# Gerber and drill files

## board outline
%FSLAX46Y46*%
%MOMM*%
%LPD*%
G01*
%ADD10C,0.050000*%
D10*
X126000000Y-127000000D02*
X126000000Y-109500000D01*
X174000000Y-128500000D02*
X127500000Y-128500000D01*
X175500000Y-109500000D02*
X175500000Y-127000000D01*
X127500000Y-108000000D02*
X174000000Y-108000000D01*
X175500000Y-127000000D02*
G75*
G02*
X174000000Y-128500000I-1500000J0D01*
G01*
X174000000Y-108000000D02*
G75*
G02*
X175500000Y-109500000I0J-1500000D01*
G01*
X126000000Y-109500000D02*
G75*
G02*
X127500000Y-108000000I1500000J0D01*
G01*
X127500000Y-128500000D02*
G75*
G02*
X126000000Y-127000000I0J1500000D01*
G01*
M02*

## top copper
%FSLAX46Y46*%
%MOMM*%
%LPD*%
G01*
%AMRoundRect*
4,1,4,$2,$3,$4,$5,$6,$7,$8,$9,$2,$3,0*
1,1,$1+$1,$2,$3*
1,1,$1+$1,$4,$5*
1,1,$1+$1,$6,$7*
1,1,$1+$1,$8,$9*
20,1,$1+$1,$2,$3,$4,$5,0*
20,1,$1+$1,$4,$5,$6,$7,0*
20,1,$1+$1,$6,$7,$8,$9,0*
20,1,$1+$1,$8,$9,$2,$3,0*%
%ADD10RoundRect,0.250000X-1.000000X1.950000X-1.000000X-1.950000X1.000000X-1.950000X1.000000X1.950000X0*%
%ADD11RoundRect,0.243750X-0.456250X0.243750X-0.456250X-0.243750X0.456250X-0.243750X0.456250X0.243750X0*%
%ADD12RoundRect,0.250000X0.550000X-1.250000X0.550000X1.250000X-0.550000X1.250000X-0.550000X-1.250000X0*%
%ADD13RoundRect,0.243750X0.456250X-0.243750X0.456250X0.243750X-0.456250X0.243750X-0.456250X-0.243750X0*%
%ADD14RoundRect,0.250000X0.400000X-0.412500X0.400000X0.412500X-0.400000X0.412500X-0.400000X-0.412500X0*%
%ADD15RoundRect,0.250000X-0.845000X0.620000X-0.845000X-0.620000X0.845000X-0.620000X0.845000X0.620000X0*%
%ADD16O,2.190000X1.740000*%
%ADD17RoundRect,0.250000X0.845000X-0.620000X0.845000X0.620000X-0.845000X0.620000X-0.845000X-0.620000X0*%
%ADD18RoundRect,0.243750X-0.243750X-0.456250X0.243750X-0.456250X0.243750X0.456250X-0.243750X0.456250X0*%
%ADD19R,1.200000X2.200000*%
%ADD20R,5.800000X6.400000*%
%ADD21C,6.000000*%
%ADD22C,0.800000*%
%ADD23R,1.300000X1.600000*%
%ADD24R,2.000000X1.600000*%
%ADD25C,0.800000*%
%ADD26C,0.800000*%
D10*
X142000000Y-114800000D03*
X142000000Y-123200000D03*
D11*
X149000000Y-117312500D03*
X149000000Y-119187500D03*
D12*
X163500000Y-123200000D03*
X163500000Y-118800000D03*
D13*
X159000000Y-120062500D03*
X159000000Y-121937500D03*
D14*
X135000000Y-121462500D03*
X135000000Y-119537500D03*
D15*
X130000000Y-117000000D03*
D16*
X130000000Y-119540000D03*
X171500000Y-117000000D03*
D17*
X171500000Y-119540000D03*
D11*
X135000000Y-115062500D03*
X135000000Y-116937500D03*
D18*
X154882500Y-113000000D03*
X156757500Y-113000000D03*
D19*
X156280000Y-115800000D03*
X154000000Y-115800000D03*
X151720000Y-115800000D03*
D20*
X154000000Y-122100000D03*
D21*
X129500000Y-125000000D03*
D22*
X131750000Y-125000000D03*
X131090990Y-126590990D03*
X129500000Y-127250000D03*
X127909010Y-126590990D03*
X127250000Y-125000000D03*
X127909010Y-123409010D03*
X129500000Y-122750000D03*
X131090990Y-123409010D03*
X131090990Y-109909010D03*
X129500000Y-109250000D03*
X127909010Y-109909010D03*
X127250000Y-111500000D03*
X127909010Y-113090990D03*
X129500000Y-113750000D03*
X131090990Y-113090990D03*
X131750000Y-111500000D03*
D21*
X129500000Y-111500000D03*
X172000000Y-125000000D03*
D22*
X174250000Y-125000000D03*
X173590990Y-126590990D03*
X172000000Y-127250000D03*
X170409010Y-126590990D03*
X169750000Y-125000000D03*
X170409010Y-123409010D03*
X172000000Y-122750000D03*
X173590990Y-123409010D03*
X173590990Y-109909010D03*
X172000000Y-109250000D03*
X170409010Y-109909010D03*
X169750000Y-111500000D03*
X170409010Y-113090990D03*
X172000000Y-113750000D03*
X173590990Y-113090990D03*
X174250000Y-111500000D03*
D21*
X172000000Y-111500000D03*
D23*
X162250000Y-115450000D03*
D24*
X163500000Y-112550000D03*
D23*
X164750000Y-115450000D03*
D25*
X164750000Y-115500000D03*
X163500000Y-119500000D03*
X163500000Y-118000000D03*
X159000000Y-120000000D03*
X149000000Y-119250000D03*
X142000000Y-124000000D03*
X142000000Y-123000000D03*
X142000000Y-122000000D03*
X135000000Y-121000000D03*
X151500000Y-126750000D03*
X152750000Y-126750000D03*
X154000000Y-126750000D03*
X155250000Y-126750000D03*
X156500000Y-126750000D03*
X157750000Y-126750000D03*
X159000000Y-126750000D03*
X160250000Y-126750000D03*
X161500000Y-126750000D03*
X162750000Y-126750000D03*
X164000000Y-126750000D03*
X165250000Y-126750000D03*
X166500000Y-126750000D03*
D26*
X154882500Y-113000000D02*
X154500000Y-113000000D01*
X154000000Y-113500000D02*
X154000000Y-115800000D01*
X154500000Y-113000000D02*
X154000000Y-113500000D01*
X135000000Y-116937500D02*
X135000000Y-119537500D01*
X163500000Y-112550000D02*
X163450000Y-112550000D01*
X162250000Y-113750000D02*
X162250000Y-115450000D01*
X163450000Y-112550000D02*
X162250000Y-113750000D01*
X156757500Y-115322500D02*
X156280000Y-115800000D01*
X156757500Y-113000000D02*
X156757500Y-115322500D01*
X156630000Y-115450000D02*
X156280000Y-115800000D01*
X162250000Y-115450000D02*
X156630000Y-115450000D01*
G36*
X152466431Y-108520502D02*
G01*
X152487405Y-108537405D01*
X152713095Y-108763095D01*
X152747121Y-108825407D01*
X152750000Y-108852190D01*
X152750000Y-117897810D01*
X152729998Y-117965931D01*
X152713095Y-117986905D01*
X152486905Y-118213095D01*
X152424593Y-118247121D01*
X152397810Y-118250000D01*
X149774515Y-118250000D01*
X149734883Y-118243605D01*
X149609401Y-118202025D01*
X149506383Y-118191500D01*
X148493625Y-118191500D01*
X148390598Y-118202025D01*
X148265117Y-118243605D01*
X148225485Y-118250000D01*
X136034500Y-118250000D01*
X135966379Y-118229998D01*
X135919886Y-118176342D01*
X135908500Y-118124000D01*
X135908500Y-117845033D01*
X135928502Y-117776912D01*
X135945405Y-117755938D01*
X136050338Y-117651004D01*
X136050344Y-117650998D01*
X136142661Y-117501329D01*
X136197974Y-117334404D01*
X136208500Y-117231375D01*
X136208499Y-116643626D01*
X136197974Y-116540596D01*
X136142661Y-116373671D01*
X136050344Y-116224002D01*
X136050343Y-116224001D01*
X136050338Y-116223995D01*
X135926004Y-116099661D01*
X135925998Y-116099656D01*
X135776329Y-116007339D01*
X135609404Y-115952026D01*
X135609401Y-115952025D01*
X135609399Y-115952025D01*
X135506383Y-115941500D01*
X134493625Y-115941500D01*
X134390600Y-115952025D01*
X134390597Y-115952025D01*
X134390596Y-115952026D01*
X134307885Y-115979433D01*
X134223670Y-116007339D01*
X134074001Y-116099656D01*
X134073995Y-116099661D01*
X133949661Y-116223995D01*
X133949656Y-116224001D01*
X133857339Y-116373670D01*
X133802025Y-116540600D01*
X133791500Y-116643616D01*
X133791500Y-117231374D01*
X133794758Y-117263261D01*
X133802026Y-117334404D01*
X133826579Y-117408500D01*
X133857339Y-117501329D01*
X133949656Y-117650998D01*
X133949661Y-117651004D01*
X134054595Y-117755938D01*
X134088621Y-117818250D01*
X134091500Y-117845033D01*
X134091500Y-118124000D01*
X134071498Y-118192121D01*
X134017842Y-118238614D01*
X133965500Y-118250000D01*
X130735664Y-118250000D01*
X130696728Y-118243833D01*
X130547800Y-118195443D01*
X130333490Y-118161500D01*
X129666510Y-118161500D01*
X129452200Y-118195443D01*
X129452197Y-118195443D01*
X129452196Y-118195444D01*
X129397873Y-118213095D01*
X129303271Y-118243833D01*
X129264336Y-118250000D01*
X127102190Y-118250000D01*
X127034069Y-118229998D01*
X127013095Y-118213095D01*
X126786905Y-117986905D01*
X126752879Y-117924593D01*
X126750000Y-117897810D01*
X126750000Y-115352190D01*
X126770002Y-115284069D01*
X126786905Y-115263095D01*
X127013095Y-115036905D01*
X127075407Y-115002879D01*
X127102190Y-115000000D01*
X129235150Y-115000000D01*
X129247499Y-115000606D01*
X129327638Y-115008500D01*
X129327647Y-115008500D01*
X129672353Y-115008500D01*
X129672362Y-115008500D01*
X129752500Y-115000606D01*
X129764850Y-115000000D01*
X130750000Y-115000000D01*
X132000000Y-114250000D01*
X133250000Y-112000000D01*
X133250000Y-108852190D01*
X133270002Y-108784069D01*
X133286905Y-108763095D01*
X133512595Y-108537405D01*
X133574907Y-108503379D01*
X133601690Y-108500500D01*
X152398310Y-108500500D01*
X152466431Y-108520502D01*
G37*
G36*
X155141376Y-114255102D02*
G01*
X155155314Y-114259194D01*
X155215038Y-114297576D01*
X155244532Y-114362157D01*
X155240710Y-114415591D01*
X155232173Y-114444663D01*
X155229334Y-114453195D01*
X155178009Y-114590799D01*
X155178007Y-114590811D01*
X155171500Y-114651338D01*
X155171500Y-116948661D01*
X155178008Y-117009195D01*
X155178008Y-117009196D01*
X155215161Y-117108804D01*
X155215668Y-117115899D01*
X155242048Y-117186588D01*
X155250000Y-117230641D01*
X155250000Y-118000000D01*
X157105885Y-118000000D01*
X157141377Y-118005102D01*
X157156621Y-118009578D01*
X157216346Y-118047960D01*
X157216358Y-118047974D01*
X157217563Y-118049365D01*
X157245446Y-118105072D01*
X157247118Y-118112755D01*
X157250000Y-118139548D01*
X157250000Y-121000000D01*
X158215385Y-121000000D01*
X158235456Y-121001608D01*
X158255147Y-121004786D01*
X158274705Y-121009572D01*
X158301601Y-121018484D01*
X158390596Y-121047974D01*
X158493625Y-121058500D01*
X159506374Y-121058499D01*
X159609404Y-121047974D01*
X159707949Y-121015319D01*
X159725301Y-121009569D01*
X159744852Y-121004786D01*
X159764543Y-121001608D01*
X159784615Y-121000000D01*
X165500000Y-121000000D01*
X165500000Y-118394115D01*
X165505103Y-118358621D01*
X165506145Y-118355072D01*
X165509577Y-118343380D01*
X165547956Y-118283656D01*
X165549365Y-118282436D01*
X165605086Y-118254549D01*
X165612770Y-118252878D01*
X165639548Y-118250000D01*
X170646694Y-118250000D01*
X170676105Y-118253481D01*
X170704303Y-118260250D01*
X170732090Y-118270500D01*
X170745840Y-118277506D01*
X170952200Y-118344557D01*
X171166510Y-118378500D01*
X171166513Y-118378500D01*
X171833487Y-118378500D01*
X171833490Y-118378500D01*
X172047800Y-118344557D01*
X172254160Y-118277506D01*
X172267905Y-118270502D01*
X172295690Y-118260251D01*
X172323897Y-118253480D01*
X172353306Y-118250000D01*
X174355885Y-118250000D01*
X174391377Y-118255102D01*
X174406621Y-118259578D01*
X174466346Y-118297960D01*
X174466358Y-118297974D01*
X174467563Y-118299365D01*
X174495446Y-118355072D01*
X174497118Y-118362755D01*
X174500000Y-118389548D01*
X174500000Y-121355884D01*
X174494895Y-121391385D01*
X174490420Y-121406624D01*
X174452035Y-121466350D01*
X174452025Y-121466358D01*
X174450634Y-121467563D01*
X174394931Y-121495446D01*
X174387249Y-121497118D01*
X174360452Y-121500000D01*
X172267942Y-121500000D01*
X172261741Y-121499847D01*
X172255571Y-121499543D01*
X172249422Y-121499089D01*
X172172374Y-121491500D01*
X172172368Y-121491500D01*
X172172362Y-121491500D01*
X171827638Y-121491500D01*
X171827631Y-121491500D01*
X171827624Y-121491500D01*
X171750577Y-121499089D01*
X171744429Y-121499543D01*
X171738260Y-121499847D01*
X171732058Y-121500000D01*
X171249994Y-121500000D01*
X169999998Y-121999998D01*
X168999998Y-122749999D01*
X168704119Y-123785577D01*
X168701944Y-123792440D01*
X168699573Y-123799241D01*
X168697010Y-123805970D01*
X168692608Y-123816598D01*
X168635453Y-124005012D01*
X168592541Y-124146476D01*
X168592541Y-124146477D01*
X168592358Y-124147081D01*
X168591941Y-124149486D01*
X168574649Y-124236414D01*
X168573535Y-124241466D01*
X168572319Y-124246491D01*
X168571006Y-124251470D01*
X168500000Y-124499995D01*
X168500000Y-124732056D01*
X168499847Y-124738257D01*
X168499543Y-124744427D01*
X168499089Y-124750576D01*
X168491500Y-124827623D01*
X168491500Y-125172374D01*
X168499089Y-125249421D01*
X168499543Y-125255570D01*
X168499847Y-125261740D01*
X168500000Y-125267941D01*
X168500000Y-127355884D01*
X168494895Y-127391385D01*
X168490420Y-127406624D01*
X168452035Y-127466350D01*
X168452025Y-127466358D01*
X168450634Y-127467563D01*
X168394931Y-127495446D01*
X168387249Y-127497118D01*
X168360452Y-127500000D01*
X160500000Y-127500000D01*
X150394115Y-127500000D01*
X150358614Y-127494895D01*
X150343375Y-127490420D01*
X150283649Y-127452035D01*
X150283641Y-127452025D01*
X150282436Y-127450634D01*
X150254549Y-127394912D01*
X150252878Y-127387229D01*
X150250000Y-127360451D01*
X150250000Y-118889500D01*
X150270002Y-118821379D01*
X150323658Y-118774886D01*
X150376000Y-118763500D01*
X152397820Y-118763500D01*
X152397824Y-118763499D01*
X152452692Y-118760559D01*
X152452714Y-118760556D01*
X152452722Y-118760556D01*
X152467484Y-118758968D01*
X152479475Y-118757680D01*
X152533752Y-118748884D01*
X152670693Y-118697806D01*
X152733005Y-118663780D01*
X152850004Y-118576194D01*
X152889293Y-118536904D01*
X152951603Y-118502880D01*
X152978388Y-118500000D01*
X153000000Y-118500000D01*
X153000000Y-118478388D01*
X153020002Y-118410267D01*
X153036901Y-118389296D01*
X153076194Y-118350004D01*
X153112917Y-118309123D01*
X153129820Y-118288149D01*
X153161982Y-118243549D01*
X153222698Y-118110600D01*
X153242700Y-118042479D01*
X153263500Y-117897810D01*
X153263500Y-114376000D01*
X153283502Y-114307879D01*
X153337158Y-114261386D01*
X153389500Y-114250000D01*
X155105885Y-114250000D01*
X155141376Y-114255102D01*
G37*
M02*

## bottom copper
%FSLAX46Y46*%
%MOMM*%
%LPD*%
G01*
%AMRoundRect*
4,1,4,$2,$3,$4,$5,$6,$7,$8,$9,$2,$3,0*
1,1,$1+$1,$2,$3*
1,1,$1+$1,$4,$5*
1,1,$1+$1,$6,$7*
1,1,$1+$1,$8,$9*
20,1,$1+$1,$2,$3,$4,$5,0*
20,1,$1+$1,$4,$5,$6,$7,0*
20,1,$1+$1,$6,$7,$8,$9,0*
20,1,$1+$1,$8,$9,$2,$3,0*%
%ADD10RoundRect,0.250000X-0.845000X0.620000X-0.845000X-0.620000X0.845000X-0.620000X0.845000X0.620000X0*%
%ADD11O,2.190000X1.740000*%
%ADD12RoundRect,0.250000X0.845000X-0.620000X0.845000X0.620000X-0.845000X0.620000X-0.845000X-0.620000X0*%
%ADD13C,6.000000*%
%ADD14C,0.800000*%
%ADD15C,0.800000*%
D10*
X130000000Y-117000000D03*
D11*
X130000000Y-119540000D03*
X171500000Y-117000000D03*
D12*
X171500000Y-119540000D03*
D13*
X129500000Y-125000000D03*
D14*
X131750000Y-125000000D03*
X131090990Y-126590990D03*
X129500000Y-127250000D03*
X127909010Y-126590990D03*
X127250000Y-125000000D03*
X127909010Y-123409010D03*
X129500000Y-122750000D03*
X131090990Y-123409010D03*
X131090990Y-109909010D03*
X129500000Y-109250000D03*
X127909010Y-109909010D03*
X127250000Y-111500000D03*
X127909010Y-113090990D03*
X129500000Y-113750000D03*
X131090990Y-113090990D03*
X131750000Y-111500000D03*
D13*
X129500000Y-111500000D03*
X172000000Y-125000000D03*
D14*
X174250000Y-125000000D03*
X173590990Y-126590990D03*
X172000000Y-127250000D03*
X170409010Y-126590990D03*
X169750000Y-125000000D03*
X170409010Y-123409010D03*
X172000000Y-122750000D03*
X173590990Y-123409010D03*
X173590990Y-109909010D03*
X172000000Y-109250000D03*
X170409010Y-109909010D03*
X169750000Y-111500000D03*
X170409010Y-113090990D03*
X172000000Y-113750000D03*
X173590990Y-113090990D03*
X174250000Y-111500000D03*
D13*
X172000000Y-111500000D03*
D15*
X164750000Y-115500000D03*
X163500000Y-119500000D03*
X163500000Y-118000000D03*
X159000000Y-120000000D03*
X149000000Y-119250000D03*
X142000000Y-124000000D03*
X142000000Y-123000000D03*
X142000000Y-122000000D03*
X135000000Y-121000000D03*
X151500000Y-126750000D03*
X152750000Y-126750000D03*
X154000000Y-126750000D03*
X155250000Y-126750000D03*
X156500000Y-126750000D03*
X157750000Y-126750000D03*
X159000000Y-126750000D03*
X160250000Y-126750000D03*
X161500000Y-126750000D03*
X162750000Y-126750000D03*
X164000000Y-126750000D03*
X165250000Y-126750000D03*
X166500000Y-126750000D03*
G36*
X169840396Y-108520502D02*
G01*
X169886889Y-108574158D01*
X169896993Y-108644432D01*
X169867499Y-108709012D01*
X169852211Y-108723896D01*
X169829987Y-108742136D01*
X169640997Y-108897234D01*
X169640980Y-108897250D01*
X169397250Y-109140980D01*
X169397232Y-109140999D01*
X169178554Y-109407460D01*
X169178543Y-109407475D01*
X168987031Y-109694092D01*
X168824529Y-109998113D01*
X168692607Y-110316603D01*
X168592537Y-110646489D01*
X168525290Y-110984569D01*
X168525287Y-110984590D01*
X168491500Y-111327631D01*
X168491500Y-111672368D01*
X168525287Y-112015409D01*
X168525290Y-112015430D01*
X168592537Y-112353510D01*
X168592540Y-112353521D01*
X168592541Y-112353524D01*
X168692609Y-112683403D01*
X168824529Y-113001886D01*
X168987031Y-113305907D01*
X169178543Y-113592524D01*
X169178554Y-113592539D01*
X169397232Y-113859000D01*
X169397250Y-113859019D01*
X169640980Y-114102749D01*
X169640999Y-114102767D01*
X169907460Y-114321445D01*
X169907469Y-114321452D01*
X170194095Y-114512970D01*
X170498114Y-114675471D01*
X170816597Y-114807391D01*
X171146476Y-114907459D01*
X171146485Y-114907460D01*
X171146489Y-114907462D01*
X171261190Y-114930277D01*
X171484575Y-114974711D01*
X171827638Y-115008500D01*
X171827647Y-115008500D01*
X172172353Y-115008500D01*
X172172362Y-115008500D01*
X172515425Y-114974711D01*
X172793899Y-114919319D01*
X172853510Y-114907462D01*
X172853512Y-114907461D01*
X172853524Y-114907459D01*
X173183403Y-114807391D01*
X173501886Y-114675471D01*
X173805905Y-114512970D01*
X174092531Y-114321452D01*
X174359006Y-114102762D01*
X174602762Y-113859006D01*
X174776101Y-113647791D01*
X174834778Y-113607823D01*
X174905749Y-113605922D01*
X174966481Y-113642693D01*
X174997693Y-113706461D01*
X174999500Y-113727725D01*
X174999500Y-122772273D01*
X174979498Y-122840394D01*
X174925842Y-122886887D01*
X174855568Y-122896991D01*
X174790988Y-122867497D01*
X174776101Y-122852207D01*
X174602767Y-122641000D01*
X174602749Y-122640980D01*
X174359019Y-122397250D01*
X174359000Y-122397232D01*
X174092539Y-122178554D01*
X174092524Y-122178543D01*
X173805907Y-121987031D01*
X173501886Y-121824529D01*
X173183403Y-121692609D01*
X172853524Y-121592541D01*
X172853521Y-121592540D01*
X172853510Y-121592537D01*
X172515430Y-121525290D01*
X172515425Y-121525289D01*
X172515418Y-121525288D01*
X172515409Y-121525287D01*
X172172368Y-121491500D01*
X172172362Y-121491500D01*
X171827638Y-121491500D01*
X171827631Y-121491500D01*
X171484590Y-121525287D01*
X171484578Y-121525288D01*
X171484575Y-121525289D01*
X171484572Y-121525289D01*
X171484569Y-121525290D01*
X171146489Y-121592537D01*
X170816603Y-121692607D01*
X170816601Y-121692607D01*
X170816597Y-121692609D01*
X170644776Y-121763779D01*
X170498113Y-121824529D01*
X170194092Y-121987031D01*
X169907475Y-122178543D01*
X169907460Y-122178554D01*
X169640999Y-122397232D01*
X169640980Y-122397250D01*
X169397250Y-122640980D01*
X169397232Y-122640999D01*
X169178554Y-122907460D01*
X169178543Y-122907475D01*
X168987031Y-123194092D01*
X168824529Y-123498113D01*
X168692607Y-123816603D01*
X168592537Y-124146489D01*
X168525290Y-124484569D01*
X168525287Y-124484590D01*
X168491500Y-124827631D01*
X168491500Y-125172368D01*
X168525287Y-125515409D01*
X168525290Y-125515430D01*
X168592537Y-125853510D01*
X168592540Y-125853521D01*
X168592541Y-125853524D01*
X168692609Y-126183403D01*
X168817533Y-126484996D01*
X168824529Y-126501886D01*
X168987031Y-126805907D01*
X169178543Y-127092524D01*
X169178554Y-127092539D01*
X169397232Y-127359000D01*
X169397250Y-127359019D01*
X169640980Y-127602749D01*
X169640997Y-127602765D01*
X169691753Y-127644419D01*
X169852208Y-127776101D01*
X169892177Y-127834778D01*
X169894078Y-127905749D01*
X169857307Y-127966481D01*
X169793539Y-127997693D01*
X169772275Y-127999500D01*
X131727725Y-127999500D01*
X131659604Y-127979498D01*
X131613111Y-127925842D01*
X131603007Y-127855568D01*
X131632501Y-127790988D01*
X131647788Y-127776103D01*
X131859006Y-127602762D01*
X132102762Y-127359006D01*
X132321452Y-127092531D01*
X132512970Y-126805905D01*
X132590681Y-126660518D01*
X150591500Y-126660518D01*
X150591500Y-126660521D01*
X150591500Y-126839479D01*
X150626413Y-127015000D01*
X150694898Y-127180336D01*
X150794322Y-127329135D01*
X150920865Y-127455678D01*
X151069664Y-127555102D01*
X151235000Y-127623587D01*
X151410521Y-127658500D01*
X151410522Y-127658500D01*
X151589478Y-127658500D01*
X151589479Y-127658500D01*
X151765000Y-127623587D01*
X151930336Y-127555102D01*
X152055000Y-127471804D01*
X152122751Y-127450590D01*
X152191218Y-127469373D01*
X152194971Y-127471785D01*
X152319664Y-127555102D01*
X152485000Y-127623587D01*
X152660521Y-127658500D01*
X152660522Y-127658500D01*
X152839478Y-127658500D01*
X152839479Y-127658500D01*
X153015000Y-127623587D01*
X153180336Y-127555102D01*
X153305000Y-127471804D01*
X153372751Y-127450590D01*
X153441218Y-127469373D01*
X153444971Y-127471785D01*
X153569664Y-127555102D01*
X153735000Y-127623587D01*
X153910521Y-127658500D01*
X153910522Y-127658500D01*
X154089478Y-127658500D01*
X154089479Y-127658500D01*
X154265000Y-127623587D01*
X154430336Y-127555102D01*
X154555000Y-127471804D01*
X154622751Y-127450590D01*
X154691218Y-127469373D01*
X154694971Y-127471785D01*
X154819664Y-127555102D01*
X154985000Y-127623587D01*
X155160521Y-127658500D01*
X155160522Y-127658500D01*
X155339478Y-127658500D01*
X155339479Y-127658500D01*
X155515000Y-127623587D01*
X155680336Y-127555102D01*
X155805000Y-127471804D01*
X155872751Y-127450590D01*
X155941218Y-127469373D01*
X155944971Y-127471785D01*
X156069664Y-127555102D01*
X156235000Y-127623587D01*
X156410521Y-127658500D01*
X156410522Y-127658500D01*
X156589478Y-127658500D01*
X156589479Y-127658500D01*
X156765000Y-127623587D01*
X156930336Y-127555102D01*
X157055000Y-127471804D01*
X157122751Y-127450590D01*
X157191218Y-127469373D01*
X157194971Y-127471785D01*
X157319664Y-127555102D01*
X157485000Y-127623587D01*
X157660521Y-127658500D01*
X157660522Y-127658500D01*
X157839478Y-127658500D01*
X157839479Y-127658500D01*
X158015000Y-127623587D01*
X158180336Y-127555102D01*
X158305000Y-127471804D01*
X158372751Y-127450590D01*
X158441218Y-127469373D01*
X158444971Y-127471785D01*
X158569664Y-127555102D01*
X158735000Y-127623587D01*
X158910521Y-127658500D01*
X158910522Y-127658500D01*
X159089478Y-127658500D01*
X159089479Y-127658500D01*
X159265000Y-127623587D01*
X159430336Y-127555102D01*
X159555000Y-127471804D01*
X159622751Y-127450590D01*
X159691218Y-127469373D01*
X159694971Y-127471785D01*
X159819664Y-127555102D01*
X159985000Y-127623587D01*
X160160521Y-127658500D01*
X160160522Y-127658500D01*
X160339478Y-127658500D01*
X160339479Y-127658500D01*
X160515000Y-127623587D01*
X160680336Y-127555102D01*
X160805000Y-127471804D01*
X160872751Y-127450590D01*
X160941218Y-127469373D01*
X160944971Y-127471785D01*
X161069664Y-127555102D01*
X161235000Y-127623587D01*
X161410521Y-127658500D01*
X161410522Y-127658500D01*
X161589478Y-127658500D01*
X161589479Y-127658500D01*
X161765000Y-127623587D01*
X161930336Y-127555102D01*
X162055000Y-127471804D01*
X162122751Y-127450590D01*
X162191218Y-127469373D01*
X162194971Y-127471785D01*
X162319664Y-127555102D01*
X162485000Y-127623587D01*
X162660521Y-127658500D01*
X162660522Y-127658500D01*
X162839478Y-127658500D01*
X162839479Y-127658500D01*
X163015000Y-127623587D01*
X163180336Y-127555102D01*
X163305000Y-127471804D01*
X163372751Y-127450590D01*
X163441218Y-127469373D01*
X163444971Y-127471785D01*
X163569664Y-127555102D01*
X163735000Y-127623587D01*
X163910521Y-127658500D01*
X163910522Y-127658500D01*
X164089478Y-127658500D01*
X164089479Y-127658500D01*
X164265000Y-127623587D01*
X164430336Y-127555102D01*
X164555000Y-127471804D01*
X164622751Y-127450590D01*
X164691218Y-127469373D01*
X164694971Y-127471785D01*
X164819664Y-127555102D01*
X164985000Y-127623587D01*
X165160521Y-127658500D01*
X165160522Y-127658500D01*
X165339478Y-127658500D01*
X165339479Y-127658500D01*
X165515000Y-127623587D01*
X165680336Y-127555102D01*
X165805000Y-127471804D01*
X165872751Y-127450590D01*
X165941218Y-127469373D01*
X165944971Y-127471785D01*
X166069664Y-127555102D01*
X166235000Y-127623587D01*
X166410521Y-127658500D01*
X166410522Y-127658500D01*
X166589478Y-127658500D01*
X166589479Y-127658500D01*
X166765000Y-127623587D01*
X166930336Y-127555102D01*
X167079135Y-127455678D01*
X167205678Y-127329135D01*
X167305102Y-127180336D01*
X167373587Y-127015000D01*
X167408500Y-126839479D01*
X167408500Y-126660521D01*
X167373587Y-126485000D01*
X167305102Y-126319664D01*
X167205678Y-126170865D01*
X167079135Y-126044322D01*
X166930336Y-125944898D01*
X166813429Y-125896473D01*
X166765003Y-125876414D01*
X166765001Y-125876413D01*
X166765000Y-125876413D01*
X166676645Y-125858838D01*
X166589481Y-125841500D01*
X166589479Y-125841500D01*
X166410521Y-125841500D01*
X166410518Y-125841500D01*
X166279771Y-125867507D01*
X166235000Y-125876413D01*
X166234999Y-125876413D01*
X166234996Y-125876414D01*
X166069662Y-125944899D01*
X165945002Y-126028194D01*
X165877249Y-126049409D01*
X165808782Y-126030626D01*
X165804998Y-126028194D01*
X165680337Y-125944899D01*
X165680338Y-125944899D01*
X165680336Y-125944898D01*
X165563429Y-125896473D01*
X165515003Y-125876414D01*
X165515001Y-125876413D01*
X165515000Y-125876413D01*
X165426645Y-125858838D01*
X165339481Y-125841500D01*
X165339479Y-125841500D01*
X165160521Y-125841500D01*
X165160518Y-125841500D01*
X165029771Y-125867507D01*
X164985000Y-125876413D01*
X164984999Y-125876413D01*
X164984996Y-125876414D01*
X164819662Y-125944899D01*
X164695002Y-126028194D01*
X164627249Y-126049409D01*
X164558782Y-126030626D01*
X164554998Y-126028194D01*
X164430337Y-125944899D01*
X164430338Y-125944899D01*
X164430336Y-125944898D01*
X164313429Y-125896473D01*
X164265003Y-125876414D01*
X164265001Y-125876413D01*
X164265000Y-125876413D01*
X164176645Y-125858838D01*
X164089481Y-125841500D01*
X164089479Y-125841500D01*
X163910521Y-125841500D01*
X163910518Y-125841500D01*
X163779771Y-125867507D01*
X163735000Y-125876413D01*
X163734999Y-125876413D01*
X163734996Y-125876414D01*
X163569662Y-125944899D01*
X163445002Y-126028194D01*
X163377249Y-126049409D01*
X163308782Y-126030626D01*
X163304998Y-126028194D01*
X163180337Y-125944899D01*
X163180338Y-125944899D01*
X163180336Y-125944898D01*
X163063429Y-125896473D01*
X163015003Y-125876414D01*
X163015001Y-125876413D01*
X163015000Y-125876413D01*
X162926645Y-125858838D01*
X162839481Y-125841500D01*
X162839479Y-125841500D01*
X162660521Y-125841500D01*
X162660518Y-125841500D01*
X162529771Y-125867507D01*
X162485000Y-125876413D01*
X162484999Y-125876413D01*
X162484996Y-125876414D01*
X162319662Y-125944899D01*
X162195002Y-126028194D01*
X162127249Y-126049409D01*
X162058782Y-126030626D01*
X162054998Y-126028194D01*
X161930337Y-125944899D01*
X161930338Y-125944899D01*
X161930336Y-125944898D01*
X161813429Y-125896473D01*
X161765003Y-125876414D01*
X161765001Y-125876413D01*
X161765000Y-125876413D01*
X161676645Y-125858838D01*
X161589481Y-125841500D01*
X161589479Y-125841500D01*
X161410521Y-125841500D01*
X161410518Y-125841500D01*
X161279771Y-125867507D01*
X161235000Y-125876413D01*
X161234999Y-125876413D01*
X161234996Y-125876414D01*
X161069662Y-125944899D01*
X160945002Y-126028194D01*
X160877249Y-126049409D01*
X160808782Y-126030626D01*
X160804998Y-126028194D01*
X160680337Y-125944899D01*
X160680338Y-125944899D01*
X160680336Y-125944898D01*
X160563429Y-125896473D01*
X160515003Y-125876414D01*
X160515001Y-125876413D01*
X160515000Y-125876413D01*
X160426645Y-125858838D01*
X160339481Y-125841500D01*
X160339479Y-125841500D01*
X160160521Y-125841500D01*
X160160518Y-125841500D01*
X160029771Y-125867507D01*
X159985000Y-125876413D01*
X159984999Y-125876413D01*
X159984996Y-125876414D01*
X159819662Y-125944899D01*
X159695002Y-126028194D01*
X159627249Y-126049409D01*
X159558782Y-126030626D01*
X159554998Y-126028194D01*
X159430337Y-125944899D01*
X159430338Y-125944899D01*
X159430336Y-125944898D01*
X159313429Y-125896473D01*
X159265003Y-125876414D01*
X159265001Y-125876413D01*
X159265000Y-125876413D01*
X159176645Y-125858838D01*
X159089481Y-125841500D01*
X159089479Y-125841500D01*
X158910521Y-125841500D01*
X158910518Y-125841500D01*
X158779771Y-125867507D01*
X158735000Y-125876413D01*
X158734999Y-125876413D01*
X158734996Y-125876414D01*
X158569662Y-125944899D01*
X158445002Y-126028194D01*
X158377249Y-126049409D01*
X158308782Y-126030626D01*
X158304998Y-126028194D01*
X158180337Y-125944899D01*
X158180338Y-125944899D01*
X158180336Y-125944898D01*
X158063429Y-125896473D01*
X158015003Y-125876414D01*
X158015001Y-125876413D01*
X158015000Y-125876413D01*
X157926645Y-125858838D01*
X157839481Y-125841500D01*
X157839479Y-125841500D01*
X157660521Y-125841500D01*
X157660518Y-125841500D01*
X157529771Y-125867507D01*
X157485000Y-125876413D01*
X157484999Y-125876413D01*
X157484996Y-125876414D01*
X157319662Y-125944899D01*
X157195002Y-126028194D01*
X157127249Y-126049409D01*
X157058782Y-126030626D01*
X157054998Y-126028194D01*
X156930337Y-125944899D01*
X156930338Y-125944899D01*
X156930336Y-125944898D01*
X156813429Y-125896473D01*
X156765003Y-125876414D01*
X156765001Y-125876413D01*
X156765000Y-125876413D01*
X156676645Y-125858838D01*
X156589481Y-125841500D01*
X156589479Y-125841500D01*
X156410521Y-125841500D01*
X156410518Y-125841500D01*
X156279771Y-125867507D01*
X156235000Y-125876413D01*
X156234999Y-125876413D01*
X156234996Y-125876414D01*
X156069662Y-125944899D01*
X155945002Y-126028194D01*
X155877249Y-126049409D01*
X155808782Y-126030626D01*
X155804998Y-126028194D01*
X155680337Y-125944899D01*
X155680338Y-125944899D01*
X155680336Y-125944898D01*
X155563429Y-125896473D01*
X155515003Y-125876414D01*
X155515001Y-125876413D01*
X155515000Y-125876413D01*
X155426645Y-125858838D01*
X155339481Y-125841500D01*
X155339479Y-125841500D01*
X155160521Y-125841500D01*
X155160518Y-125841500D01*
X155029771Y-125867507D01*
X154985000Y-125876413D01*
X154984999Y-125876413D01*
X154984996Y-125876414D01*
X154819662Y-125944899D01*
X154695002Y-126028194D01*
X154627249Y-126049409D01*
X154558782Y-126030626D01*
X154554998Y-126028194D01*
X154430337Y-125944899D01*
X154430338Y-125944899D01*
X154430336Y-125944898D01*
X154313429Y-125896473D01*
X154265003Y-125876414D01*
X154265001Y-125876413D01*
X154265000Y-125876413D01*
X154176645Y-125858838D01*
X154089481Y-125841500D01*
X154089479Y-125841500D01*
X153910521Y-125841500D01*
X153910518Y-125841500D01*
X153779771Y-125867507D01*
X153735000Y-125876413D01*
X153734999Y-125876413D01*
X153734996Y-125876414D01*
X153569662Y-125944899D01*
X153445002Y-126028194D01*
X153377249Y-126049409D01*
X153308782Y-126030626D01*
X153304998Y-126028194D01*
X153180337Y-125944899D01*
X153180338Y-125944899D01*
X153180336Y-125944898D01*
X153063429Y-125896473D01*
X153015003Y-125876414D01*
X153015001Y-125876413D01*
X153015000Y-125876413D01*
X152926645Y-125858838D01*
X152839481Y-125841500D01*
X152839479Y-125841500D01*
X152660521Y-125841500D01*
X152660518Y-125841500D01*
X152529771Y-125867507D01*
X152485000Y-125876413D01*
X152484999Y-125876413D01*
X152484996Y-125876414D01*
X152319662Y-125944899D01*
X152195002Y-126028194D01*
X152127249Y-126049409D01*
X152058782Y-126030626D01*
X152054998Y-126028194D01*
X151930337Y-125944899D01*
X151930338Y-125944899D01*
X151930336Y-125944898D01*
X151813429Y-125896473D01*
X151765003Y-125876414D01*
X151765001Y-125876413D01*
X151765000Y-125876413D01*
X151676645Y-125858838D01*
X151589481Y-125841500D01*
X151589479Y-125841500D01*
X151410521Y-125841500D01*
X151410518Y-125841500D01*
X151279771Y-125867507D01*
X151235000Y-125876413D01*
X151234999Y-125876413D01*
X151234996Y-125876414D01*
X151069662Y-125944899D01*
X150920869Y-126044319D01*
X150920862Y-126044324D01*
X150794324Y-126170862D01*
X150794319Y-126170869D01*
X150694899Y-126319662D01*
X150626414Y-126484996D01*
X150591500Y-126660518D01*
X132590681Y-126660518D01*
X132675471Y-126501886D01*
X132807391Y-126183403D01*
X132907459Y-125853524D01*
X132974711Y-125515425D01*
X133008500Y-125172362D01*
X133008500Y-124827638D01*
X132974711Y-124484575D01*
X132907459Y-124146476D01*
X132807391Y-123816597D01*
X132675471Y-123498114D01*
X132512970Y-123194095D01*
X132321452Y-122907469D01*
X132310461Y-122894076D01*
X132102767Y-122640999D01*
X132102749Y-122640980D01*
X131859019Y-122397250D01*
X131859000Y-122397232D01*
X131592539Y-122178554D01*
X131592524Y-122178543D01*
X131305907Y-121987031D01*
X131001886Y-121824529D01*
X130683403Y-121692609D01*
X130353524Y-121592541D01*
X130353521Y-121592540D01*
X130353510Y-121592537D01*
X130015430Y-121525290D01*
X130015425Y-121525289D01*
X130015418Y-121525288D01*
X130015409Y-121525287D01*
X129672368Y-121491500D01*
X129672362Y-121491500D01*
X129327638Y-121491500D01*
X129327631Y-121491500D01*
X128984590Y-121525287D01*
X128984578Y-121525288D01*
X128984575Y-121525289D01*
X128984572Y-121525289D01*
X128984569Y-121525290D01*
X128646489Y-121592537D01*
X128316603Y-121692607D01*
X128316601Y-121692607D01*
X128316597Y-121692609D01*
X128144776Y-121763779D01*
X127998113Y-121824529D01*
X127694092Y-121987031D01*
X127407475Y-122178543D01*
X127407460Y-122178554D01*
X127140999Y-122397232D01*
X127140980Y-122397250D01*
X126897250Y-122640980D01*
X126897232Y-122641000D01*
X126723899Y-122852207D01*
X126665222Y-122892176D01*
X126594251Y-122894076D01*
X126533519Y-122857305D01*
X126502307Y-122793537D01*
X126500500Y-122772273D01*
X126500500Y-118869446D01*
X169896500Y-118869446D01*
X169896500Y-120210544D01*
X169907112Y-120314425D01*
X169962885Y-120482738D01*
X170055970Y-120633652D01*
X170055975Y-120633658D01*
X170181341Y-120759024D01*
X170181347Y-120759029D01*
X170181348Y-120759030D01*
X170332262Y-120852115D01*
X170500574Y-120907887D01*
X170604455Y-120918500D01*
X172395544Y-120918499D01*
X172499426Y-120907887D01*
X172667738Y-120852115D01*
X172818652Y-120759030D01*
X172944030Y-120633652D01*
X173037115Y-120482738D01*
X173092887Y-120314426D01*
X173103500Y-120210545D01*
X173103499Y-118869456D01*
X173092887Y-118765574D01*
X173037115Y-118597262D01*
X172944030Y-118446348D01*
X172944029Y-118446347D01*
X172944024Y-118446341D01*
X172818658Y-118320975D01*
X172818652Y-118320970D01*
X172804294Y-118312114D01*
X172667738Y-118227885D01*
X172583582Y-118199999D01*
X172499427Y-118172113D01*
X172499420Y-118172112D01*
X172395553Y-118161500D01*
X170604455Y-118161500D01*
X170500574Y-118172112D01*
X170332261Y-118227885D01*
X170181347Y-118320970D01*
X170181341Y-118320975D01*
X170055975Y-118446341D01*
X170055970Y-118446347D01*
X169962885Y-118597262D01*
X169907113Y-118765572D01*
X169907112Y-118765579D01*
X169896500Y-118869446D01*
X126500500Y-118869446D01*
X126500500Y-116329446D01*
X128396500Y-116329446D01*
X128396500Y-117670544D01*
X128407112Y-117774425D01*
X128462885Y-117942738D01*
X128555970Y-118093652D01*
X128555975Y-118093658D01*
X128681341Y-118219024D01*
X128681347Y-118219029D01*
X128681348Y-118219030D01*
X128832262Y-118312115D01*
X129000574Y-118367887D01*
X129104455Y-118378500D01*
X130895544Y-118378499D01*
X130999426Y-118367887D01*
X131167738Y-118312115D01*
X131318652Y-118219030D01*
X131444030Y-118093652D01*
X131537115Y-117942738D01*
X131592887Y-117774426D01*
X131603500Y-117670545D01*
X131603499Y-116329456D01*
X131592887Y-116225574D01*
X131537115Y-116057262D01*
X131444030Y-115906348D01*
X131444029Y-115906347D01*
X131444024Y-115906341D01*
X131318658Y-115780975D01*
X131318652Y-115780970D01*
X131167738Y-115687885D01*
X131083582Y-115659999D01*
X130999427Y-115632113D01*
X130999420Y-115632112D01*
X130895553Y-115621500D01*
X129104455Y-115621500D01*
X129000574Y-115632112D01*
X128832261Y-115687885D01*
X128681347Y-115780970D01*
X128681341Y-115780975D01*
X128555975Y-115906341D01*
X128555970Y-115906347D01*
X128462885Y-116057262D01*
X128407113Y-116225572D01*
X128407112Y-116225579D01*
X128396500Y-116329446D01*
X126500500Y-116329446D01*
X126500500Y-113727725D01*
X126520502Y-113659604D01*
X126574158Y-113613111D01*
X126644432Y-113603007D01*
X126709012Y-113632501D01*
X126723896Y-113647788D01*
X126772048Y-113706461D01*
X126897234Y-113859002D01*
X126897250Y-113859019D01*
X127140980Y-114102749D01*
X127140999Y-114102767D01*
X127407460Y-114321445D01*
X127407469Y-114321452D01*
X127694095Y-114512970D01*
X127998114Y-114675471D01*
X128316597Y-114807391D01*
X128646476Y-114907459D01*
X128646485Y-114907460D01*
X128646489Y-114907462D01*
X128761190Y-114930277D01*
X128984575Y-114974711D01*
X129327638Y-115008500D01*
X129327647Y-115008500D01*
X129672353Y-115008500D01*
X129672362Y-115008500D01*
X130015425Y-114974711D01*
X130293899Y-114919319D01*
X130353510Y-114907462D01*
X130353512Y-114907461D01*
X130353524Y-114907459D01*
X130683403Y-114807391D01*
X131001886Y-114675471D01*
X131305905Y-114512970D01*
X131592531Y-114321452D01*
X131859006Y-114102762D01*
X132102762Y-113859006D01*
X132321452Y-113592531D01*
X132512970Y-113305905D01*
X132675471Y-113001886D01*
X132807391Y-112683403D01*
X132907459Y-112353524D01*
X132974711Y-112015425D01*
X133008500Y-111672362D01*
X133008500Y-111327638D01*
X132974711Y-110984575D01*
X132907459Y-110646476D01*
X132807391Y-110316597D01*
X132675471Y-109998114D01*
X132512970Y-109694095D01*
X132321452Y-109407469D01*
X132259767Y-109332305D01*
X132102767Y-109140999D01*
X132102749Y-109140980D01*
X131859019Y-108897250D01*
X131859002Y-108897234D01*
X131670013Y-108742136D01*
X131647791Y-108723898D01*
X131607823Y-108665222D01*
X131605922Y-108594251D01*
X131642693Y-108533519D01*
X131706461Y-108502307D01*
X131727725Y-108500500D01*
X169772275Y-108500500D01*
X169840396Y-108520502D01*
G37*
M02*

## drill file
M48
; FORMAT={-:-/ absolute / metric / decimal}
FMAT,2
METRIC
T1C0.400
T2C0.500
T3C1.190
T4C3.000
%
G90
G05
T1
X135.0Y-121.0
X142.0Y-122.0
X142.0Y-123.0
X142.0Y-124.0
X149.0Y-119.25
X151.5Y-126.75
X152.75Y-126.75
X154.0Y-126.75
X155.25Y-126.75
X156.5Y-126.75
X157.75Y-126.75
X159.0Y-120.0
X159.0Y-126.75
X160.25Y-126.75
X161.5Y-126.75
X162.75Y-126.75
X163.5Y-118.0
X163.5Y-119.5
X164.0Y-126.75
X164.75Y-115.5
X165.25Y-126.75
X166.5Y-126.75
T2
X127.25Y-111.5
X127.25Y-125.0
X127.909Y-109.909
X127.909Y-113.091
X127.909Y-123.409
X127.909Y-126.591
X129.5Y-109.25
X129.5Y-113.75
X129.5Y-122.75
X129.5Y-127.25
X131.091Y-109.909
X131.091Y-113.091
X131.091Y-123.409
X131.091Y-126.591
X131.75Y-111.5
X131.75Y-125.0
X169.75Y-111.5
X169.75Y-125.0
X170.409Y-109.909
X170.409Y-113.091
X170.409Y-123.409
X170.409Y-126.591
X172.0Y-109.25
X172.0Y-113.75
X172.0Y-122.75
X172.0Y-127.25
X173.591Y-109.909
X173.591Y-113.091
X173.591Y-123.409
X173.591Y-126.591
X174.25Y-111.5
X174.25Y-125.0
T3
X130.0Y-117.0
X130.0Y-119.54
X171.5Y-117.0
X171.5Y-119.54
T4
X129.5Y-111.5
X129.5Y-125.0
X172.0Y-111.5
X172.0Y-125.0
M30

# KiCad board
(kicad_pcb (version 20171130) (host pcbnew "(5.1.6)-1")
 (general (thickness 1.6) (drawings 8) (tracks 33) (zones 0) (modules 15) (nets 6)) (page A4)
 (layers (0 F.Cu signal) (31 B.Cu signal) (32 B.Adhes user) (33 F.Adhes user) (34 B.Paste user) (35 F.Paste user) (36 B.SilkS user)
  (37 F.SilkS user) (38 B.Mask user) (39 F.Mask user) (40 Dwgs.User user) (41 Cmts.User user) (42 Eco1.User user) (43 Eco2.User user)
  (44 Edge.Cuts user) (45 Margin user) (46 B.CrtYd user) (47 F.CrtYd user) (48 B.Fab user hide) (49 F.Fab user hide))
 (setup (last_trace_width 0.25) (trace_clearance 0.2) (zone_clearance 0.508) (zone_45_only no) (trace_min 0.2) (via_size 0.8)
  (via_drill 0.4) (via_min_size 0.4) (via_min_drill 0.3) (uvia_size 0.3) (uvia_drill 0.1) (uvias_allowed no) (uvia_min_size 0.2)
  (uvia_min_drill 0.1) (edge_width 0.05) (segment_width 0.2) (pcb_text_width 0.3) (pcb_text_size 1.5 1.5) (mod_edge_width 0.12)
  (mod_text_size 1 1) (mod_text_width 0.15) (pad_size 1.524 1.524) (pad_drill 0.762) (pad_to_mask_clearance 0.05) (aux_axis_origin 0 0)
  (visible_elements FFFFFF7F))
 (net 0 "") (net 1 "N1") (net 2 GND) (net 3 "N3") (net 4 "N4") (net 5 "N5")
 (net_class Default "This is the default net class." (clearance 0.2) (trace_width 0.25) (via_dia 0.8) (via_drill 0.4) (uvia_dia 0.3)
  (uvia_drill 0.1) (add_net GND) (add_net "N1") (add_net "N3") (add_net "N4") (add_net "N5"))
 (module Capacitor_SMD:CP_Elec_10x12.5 (layer F.Cu) (at 142 119 270)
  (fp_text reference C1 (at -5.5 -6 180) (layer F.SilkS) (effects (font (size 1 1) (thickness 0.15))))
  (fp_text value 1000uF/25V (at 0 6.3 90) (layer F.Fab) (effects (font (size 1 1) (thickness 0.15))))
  (pad 1 smd roundrect (at -4.2 0 270) (size 4.4 2.5) (layers F.Cu F.Paste F.Mask) (roundrect_rratio 0.1) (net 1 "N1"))
  (pad 2 smd roundrect (at 4.2 0 270) (size 4.4 2.5) (layers F.Cu F.Paste F.Mask) (roundrect_rratio 0.1) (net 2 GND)))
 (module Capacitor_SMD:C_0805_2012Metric (layer F.Cu) (at 149 118.25 270)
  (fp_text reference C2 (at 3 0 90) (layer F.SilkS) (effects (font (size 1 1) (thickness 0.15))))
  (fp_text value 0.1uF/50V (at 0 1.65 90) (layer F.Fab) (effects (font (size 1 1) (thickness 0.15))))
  (pad 1 smd roundrect (at -0.9375 0 270) (size 0.975 1.4) (layers F.Cu F.Paste F.Mask) (roundrect_rratio 0.25) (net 1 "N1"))
  (pad 2 smd roundrect (at 0.9375 0 270) (size 0.975 1.4) (layers F.Cu F.Paste F.Mask) (roundrect_rratio 0.25) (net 2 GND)))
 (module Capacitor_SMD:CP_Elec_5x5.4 (layer F.Cu) (at 163.5 121 90)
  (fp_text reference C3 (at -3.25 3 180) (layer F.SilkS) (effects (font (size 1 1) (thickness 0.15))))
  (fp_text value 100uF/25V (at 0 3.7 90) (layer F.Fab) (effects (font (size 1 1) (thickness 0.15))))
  (pad 1 smd roundrect (at -2.2 0 90) (size 3 1.6) (layers F.Cu F.Paste F.Mask) (roundrect_rratio 0.15625) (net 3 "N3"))
  (pad 2 smd roundrect (at 2.2 0 90) (size 3 1.6) (layers F.Cu F.Paste F.Mask) (roundrect_rratio 0.15625) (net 2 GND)))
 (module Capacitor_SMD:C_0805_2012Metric (layer F.Cu) (at 159 121 90)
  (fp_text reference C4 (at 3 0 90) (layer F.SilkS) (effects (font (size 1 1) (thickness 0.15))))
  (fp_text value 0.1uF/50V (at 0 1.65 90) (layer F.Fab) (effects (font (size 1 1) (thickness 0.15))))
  (pad 2 smd roundrect (at 0.9375 0 90) (size 0.975 1.4) (layers F.Cu F.Paste F.Mask) (roundrect_rratio 0.25) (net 2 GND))
  (pad 1 smd roundrect (at -0.9375 0 90) (size 0.975 1.4) (layers F.Cu F.Paste F.Mask) (roundrect_rratio 0.25) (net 3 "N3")))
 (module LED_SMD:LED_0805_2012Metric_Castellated (layer F.Cu) (at 135 120.5 90)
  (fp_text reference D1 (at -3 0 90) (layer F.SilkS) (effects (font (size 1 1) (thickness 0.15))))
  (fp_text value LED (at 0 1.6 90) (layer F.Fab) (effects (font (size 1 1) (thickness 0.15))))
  (pad 1 smd roundrect (at -0.9625 0 90) (size 1.325 1.3) (layers F.Cu F.Paste F.Mask) (roundrect_rratio 0.192308) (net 2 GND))
  (pad 2 smd roundrect (at 0.9625 0 90) (size 1.325 1.3) (layers F.Cu F.Paste F.Mask) (roundrect_rratio 0.192308) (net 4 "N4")))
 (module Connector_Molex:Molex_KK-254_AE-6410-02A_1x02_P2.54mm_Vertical (layer F.Cu) (at 130 117 270)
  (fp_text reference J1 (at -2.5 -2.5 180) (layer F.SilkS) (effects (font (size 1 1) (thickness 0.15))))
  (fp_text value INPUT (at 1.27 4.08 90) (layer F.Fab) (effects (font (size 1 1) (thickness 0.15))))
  (pad 1 thru_hole roundrect (at 0 0 270) (size 1.74 2.19) (drill 1.19) (layers *.Cu *.Mask) (roundrect_rratio 0.143678) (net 1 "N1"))
  (pad 2 thru_hole oval (at 2.54 0 270) (size 1.74 2.19) (drill 1.19) (layers *.Cu *.Mask) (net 2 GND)))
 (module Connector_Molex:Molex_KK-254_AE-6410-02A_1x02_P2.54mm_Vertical (layer F.Cu) (at 171.5 119.54 90)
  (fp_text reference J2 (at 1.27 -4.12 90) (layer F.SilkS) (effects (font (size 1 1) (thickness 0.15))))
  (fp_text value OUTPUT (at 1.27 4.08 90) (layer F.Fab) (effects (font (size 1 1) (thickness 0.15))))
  (pad 2 thru_hole oval (at 2.54 0 90) (size 1.74 2.19) (drill 1.19) (layers *.Cu *.Mask) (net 2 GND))
  (pad 1 thru_hole roundrect (at 0 0 90) (size 1.74 2.19) (drill 1.19) (layers *.Cu *.Mask) (roundrect_rratio 0.143678) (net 3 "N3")))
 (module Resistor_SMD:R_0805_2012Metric (layer F.Cu) (at 135 116 270)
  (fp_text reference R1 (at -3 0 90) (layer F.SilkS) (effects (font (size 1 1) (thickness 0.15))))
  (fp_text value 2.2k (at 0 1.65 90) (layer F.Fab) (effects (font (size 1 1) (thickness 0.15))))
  (pad 1 smd roundrect (at -0.9375 0 270) (size 0.975 1.4) (layers F.Cu F.Paste F.Mask) (roundrect_rratio 0.25) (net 1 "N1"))
  (pad 2 smd roundrect (at 0.9375 0 270) (size 0.975 1.4) (layers F.Cu F.Paste F.Mask) (roundrect_rratio 0.25) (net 4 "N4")))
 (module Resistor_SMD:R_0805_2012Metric (layer F.Cu) (at 155.82 113)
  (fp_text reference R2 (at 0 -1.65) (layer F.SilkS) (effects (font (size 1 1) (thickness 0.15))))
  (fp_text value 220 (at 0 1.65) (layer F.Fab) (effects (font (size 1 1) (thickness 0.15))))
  (pad 1 smd roundrect (at -0.9375 0) (size 0.975 1.4) (layers F.Cu F.Paste F.Mask) (roundrect_rratio 0.25) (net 3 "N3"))
  (pad 2 smd roundrect (at 0.9375 0) (size 0.975 1.4) (layers F.Cu F.Paste F.Mask) (roundrect_rratio 0.25) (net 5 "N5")))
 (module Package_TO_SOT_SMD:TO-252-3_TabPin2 (layer F.Cu) (at 154 120 270)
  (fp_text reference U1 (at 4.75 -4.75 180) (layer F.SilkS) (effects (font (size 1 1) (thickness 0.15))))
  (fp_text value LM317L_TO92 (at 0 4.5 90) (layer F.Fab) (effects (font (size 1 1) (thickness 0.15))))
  (pad 1 smd rect (at -4.2 -2.28 270) (size 2.2 1.2) (layers F.Cu F.Paste F.Mask) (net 5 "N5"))
  (pad 2 smd rect (at -4.2 0 270) (size 2.2 1.2) (layers F.Cu F.Paste F.Mask) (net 3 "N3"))
  (pad 3 smd rect (at -4.2 2.28 270) (size 2.2 1.2) (layers F.Cu F.Paste F.Mask) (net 1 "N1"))
  (pad 2 smd rect (at 2.1 0 270) (size 6.4 5.8) (layers F.Cu F.Mask) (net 3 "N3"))
  (pad "" smd rect (at 3.775 1.525 270) (size 3.05 2.75) (layers F.Paste))
  (pad "" smd rect (at 0.425 -1.525 270) (size 3.05 2.75) (layers F.Paste))
  (pad "" smd rect (at 3.775 -1.525 270) (size 3.05 2.75) (layers F.Paste))
  (pad "" smd rect (at 0.425 1.525 270) (size 3.05 2.75) (layers F.Paste)))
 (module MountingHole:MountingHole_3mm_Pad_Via (layer F.Cu) (at 129.5 125)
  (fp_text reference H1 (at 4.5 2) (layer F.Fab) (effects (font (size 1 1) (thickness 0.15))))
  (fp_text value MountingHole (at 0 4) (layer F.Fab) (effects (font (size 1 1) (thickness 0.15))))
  (pad 1 thru_hole circle (at 0 0) (size 6 6) (drill 3) (layers *.Cu *.Mask))
  (pad 1 thru_hole circle (at 2.25 0) (size 0.8 0.8) (drill 0.5) (layers *.Cu *.Mask))
  (pad 1 thru_hole circle (at 1.59099 1.59099) (size 0.8 0.8) (drill 0.5) (layers *.Cu *.Mask))
  (pad 1 thru_hole circle (at 0 2.25) (size 0.8 0.8) (drill 0.5) (layers *.Cu *.Mask))
  (pad 1 thru_hole circle (at -1.59099 1.59099) (size 0.8 0.8) (drill 0.5) (layers *.Cu *.Mask))
  (pad 1 thru_hole circle (at -2.25 0) (size 0.8 0.8) (drill 0.5) (layers *.Cu *.Mask))
  (pad 1 thru_hole circle (at -1.59099 -1.59099) (size 0.8 0.8) (drill 0.5) (layers *.Cu *.Mask))
  (pad 1 thru_hole circle (at 0 -2.25) (size 0.8 0.8) (drill 0.5) (layers *.Cu *.Mask))
  (pad 1 thru_hole circle (at 1.59099 -1.59099) (size 0.8 0.8) (drill 0.5) (layers *.Cu *.Mask)))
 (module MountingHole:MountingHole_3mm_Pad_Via (layer F.Cu) (at 129.5 111.5)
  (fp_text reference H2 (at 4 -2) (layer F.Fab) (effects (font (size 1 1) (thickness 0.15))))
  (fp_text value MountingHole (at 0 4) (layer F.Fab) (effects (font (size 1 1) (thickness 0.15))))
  (pad 1 thru_hole circle (at 1.59099 -1.59099) (size 0.8 0.8) (drill 0.5) (layers *.Cu *.Mask))
  (pad 1 thru_hole circle (at 0 -2.25) (size 0.8 0.8) (drill 0.5) (layers *.Cu *.Mask))
  (pad 1 thru_hole circle (at -1.59099 -1.59099) (size 0.8 0.8) (drill 0.5) (layers *.Cu *.Mask))
  (pad 1 thru_hole circle (at -2.25 0) (size 0.8 0.8) (drill 0.5) (layers *.Cu *.Mask))
  (pad 1 thru_hole circle (at -1.59099 1.59099) (size 0.8 0.8) (drill 0.5) (layers *.Cu *.Mask))
  (pad 1 thru_hole circle (at 0 2.25) (size 0.8 0.8) (drill 0.5) (layers *.Cu *.Mask))
  (pad 1 thru_hole circle (at 1.59099 1.59099) (size 0.8 0.8) (drill 0.5) (layers *.Cu *.Mask))
  (pad 1 thru_hole circle (at 2.25 0) (size 0.8 0.8) (drill 0.5) (layers *.Cu *.Mask))
  (pad 1 thru_hole circle (at 0 0) (size 6 6) (drill 3) (layers *.Cu *.Mask)))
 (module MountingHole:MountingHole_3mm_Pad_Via (layer F.Cu) (at 172 125)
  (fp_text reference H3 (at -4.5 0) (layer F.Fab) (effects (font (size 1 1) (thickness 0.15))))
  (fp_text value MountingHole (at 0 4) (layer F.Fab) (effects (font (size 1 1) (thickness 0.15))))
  (pad 1 thru_hole circle (at 0 0) (size 6 6) (drill 3) (layers *.Cu *.Mask))
  (pad 1 thru_hole circle (at 2.25 0) (size 0.8 0.8) (drill 0.5) (layers *.Cu *.Mask))
  (pad 1 thru_hole circle (at 1.59099 1.59099) (size 0.8 0.8) (drill 0.5) (layers *.Cu *.Mask))
  (pad 1 thru_hole circle (at 0 2.25) (size 0.8 0.8) (drill 0.5) (layers *.Cu *.Mask))
  (pad 1 thru_hole circle (at -1.59099 1.59099) (size 0.8 0.8) (drill 0.5) (layers *.Cu *.Mask))
  (pad 1 thru_hole circle (at -2.25 0) (size 0.8 0.8) (drill 0.5) (layers *.Cu *.Mask))
  (pad 1 thru_hole circle (at -1.59099 -1.59099) (size 0.8 0.8) (drill 0.5) (layers *.Cu *.Mask))
  (pad 1 thru_hole circle (at 0 -2.25) (size 0.8 0.8) (drill 0.5) (layers *.Cu *.Mask))
  (pad 1 thru_hole circle (at 1.59099 -1.59099) (size 0.8 0.8) (drill 0.5) (layers *.Cu *.Mask)))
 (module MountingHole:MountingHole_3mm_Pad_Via (layer F.Cu) (at 172 111.5)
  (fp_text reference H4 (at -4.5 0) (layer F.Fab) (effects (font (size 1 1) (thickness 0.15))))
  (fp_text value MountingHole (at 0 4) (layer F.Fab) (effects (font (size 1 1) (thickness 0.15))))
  (pad 1 thru_hole circle (at 1.59099 -1.59099) (size 0.8 0.8) (drill 0.5) (layers *.Cu *.Mask))
  (pad 1 thru_hole circle (at 0 -2.25) (size 0.8 0.8) (drill 0.5) (layers *.Cu *.Mask))
  (pad 1 thru_hole circle (at -1.59099 -1.59099) (size 0.8 0.8) (drill 0.5) (layers *.Cu *.Mask))
  (pad 1 thru_hole circle (at -2.25 0) (size 0.8 0.8) (drill 0.5) (layers *.Cu *.Mask))
  (pad 1 thru_hole circle (at -1.59099 1.59099) (size 0.8 0.8) (drill 0.5) (layers *.Cu *.Mask))
  (pad 1 thru_hole circle (at 0 2.25) (size 0.8 0.8) (drill 0.5) (layers *.Cu *.Mask))
  (pad 1 thru_hole circle (at 1.59099 1.59099) (size 0.8 0.8) (drill 0.5) (layers *.Cu *.Mask))
  (pad 1 thru_hole circle (at 2.25 0) (size 0.8 0.8) (drill 0.5) (layers *.Cu *.Mask))
  (pad 1 thru_hole circle (at 0 0) (size 6 6) (drill 3) (layers *.Cu *.Mask)))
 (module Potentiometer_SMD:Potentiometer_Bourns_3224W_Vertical (layer F.Cu) (at 163.5 114 180)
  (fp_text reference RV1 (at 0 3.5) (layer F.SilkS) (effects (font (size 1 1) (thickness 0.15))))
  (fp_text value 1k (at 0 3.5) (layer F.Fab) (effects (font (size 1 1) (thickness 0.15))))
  (pad 1 smd rect (at 1.25 -1.45 180) (size 1.3 1.6) (layers F.Cu F.Paste F.Mask) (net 5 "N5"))
  (pad 2 smd rect (at 0 1.45 180) (size 2 1.6) (layers F.Cu F.Paste F.Mask) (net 5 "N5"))
  (pad 3 smd rect (at -1.25 -1.45 180) (size 1.3 1.6) (layers F.Cu F.Paste F.Mask) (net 2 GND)))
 (gr_line (start 126 127) (end 126 109.5) (layer Edge.Cuts) (width 0.05))
 (gr_line (start 174 128.5) (end 127.5 128.5) (layer Edge.Cuts) (width 0.05))
 (gr_line (start 175.5 109.5) (end 175.5 127) (layer Edge.Cuts) (width 0.05))
 (gr_line (start 127.5 108) (end 174 108) (layer Edge.Cuts) (width 0.05))
 (gr_arc (start 174 127) (end 174 128.5) (angle -90) (layer Edge.Cuts) (width 0.05))
 (gr_arc (start 174 109.5) (end 175.5 109.5) (angle -90) (layer Edge.Cuts) (width 0.05))
 (gr_arc (start 127.5 109.5) (end 127.5 108) (angle -90) (layer Edge.Cuts) (width 0.05))
 (gr_arc (start 127.5 127) (end 126 127) (angle -90) (layer Edge.Cuts) (width 0.05))
 (via (at 164.75 115.5) (size 0.8) (drill 0.4) (layers F.Cu B.Cu) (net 2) (status 30))
 (via (at 163.5 119.5) (size 0.8) (drill 0.4) (layers F.Cu B.Cu) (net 2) (status 30))
 (via (at 163.5 118) (size 0.8) (drill 0.4) (layers F.Cu B.Cu) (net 2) (status 30))
 (via (at 159 120) (size 0.8) (drill 0.4) (layers F.Cu B.Cu) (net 2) (status 30))
 (via (at 149 119.25) (size 0.8) (drill 0.4) (layers F.Cu B.Cu) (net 2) (status 30))
 (via (at 142 124) (size 0.8) (drill 0.4) (layers F.Cu B.Cu) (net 2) (status 30))
 (via (at 142 123) (size 0.8) (drill 0.4) (layers F.Cu B.Cu) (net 2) (status 30))
 (via (at 142 122) (size 0.8) (drill 0.4) (layers F.Cu B.Cu) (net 2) (status 30))
 (via (at 135 121) (size 0.8) (drill 0.4) (layers F.Cu B.Cu) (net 2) (status 30))
 (segment (start 154.8825 113) (end 154.5 113) (width 0.8) (layer F.Cu) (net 3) (status 30))
 (segment (start 154 113.5) (end 154 115.8) (width 0.8) (layer F.Cu) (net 3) (status 20))
 (segment (start 154.5 113) (end 154 113.5) (width 0.8) (layer F.Cu) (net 3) (status 10))
 (via (at 151.5 126.75) (size 0.8) (drill 0.4) (layers F.Cu B.Cu) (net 3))
 (via (at 152.75 126.75) (size 0.8) (drill 0.4) (layers F.Cu B.Cu) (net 3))
 (via (at 154 126.75) (size 0.8) (drill 0.4) (layers F.Cu B.Cu) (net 3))
 (via (at 155.25 126.75) (size 0.8) (drill 0.4) (layers F.Cu B.Cu) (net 3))
 (via (at 156.5 126.75) (size 0.8) (drill 0.4) (layers F.Cu B.Cu) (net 3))
 (via (at 157.75 126.75) (size 0.8) (drill 0.4) (layers F.Cu B.Cu) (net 3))
 (via (at 159 126.75) (size 0.8) (drill 0.4) (layers F.Cu B.Cu) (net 3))
 (via (at 160.25 126.75) (size 0.8) (drill 0.4) (layers F.Cu B.Cu) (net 3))
 (via (at 161.5 126.75) (size 0.8) (drill 0.4) (layers F.Cu B.Cu) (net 3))
 (via (at 162.75 126.75) (size 0.8) (drill 0.4) (layers F.Cu B.Cu) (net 3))
 (via (at 164 126.75) (size 0.8) (drill 0.4) (layers F.Cu B.Cu) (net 3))
 (via (at 165.25 126.75) (size 0.8) (drill 0.4) (layers F.Cu B.Cu) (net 3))
 (via (at 166.5 126.75) (size 0.8) (drill 0.4) (layers F.Cu B.Cu) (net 3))
 (segment (start 135 116.9375) (end 135 119.5375) (width 0.8) (layer F.Cu) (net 4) (status 30))
 (segment (start 163.5 112.55) (end 163.45 112.55) (width 0.8) (layer F.Cu) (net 5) (status 30))
 (segment (start 162.25 113.75) (end 162.25 115.45) (width 0.8) (layer F.Cu) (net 5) (status 20))
 (segment (start 163.45 112.55) (end 162.25 113.75) (width 0.8) (layer F.Cu) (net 5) (status 10))
 (segment (start 156.7575 115.3225) (end 156.28 115.8) (width 0.8) (layer F.Cu) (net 5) (status 30))
 (segment (start 156.7575 113) (end 156.7575 115.3225) (width 0.8) (layer F.Cu) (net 5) (status 30))
 (segment (start 156.63 115.45) (end 156.28 115.8) (width 0.8) (layer F.Cu) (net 5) (status 30))
 (segment (start 162.25 115.45) (end 156.63 115.45) (width 0.8) (layer F.Cu) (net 5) (status 30))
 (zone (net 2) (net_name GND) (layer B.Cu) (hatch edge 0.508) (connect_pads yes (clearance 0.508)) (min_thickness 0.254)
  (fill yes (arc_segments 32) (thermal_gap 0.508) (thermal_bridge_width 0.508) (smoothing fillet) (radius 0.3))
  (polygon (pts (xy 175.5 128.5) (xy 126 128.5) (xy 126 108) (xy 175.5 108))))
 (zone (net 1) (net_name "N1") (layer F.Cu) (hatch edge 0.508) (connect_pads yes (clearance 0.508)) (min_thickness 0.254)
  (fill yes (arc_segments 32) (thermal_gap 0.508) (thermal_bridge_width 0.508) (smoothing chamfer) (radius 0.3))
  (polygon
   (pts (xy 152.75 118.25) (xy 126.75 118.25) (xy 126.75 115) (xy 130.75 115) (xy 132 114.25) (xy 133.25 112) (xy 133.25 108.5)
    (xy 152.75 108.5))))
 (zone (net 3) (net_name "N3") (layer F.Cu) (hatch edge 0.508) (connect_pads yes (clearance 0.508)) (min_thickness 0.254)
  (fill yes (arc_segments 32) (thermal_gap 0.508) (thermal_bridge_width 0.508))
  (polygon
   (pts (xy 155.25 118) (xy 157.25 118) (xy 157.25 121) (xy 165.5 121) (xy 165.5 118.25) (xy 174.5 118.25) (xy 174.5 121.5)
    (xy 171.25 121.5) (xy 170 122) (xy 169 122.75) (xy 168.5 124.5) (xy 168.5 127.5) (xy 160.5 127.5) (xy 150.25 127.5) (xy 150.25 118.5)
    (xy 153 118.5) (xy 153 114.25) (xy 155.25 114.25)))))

